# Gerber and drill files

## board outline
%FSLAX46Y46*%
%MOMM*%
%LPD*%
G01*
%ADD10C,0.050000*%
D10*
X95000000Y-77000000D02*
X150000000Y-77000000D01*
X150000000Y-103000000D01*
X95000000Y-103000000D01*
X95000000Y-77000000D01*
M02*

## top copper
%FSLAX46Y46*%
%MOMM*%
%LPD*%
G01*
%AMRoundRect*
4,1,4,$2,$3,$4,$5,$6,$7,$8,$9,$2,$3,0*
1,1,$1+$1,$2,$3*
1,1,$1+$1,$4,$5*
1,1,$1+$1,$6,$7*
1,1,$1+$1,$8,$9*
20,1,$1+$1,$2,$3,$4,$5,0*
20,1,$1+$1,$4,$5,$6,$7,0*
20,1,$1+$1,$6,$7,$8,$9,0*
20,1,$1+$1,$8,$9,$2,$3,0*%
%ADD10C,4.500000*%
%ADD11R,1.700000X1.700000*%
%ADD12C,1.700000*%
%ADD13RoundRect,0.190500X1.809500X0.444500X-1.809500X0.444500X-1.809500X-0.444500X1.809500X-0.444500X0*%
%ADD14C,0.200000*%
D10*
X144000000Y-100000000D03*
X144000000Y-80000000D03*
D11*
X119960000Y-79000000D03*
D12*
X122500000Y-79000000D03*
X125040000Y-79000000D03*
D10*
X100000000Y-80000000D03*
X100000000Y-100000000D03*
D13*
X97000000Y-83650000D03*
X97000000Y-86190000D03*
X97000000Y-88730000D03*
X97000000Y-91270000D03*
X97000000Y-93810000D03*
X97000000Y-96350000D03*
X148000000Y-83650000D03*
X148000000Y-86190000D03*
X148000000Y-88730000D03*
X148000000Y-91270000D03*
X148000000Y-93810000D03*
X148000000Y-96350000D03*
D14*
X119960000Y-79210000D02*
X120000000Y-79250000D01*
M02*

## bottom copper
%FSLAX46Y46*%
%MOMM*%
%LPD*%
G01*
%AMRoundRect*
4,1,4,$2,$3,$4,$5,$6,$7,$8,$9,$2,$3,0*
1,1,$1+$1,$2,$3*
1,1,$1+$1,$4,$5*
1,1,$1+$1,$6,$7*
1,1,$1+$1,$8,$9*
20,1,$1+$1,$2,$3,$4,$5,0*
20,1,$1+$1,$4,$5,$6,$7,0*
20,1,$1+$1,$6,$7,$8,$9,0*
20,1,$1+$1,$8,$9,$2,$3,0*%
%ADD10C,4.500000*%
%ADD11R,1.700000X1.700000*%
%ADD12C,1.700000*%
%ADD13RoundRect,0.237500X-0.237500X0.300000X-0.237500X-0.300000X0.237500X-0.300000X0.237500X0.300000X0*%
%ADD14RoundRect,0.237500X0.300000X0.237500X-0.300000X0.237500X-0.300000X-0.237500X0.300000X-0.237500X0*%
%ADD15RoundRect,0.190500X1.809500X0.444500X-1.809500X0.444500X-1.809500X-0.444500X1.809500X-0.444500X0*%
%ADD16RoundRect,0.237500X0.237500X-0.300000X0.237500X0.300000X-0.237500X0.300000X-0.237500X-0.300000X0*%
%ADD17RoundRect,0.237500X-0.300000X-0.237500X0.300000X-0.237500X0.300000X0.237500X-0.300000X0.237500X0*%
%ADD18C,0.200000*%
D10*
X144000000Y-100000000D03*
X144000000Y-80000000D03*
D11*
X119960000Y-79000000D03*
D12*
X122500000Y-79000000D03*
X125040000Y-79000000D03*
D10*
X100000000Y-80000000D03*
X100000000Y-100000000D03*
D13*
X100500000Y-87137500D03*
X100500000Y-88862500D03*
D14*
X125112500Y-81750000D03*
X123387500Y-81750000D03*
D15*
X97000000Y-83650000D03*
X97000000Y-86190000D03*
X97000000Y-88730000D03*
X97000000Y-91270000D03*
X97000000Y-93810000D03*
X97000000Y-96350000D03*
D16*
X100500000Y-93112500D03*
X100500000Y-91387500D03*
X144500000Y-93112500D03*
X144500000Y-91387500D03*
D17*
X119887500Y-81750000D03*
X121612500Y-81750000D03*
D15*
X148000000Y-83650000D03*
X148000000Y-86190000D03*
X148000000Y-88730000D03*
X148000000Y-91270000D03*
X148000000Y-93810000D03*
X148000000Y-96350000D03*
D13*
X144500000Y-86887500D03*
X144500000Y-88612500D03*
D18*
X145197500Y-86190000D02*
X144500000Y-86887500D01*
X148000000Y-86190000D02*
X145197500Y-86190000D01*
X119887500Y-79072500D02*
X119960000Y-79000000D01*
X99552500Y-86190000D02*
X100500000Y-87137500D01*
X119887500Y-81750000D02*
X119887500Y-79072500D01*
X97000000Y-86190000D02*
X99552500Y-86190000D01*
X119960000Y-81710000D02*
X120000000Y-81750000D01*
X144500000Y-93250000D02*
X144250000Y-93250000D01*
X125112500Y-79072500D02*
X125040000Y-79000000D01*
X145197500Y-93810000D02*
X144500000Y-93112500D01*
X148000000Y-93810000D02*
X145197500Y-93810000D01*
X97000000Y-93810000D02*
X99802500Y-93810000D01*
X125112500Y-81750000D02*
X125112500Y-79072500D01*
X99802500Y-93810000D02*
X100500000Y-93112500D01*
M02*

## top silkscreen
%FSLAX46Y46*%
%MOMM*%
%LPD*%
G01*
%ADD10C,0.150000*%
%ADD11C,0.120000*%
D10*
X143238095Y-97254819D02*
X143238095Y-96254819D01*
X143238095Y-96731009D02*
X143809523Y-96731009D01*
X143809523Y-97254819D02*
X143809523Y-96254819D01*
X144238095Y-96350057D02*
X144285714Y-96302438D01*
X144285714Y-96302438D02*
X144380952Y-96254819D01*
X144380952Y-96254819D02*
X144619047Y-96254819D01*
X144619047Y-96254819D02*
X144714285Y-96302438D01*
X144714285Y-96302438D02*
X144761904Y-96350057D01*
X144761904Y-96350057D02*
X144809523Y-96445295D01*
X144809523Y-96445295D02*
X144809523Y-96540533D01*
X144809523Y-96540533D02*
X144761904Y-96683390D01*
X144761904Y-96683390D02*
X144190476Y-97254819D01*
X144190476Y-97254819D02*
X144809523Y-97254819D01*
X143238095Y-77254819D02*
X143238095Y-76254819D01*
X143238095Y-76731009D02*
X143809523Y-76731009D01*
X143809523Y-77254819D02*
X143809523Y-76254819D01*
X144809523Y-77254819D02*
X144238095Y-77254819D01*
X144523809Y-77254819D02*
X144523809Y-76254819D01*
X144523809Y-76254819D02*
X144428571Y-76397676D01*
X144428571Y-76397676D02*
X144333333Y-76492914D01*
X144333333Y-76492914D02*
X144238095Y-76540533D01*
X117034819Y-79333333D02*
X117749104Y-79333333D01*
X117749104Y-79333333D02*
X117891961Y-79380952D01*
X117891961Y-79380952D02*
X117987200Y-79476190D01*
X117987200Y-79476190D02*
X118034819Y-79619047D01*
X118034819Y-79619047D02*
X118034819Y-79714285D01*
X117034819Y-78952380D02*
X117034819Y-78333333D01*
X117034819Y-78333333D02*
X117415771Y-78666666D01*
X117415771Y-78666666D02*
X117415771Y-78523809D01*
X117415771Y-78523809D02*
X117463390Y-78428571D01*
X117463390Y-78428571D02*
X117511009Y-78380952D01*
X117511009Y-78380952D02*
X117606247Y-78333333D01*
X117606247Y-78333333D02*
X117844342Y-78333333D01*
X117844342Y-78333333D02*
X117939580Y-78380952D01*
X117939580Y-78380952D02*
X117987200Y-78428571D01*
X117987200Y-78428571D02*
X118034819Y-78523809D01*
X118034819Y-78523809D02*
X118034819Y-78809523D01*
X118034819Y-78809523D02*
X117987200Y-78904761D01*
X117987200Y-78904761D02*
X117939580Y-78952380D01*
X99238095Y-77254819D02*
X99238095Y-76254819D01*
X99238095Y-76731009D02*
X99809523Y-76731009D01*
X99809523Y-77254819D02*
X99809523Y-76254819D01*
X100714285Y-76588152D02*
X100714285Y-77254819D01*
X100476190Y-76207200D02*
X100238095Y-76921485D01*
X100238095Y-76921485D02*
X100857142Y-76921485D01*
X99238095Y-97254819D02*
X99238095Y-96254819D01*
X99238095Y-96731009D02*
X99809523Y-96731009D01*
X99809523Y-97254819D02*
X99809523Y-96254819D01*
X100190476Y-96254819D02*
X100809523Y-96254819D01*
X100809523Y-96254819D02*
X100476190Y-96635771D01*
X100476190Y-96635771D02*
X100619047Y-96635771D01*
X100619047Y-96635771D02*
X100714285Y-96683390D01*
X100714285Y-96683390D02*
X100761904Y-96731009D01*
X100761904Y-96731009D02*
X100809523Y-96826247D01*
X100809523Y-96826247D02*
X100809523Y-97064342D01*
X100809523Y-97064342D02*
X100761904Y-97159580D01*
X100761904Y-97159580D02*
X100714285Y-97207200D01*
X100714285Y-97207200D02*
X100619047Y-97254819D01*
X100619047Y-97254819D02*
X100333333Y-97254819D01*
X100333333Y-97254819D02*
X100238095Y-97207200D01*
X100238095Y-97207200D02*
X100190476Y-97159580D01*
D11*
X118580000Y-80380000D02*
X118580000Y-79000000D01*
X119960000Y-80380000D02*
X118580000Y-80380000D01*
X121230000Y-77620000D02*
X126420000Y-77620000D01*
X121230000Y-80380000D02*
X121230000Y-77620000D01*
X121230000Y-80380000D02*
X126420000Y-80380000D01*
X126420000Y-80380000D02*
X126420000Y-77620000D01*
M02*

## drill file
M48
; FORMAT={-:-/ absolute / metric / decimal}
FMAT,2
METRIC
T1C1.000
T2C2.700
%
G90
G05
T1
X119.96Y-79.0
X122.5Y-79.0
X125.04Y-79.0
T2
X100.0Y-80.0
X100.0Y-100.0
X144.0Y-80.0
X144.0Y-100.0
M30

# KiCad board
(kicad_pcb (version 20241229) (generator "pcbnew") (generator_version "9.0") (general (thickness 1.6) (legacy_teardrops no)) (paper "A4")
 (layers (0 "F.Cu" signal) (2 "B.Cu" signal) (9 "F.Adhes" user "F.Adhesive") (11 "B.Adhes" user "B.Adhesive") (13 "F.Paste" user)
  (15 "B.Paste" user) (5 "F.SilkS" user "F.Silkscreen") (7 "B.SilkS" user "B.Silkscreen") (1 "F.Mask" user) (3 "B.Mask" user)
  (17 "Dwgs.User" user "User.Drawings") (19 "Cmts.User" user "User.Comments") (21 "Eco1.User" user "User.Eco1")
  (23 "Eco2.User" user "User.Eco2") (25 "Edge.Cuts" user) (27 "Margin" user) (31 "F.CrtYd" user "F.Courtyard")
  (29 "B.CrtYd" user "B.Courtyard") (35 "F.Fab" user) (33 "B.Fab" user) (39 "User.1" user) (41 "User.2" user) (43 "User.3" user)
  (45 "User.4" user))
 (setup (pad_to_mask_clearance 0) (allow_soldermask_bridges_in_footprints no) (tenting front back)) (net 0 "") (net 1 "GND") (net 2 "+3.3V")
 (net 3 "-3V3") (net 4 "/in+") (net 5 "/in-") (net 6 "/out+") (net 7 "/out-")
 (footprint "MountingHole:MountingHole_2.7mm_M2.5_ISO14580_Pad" (layer "F.Cu") (at 144 100)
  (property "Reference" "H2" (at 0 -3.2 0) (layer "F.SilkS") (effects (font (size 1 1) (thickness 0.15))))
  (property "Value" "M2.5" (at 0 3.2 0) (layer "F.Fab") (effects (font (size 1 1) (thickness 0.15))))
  (pad "1" thru_hole circle (at 0 0) (size 4.5 4.5) (drill 2.7) (layers "*.Cu" "*.Mask") (remove_unused_layers no) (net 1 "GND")
   (zone_connect 2)))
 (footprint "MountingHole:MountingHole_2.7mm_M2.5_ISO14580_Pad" (layer "F.Cu") (at 144 80)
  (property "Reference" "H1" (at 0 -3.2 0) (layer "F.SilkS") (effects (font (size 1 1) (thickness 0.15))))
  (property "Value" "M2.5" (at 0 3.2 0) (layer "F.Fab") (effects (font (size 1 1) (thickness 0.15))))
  (pad "1" thru_hole circle (at 0 0) (size 4.5 4.5) (drill 2.7) (layers "*.Cu" "*.Mask") (remove_unused_layers no) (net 1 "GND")
   (zone_connect 2)))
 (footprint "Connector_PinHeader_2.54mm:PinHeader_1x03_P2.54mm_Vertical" (layer "F.Cu") (at 119.96 79 90)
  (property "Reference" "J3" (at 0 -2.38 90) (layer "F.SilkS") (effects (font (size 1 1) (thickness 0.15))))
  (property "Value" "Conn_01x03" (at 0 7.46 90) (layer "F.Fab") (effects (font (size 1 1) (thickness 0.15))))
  (fp_line (start -1.38 -1.38) (end 0 -1.38) (stroke (width 0.12) (type solid)) (layer "F.SilkS"))
  (fp_line (start -1.38 0) (end -1.38 -1.38) (stroke (width 0.12) (type solid)) (layer "F.SilkS"))
  (fp_line (start 1.38 1.27) (end 1.38 6.46) (stroke (width 0.12) (type solid)) (layer "F.SilkS"))
  (fp_line (start -1.38 1.27) (end 1.38 1.27) (stroke (width 0.12) (type solid)) (layer "F.SilkS"))
  (fp_line (start -1.38 1.27) (end -1.38 6.46) (stroke (width 0.12) (type solid)) (layer "F.SilkS"))
  (fp_line (start -1.38 6.46) (end 1.38 6.46) (stroke (width 0.12) (type solid)) (layer "F.SilkS"))
  (pad "1" thru_hole rect (at 0 0 90) (size 1.7 1.7) (drill 1) (layers "*.Cu" "*.Mask") (remove_unused_layers no) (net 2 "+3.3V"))
  (pad "2" thru_hole circle (at 0 2.54 90) (size 1.7 1.7) (drill 1) (layers "*.Cu" "*.Mask") (remove_unused_layers no) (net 1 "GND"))
  (pad "3" thru_hole circle (at 0 5.08 90) (size 1.7 1.7) (drill 1) (layers "*.Cu" "*.Mask") (remove_unused_layers no) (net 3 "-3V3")))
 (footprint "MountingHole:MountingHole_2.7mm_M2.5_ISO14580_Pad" (layer "F.Cu") (at 100 80)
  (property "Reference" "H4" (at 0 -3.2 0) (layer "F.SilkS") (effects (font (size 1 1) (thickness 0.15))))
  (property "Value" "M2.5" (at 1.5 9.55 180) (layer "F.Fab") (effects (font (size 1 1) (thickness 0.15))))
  (pad "1" thru_hole circle (at 0 0) (size 4.5 4.5) (drill 2.7) (layers "*.Cu" "*.Mask") (remove_unused_layers no) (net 1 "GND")
   (zone_connect 2)))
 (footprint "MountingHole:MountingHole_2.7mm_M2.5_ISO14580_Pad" (layer "F.Cu") (at 100 100)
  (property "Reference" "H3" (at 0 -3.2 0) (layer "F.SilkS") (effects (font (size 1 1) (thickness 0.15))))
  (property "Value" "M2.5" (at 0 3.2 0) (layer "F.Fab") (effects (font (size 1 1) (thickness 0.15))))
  (pad "1" thru_hole circle (at 0 0) (size 4.5 4.5) (drill 2.7) (layers "*.Cu" "*.Mask") (remove_unused_layers no) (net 1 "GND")
   (zone_connect 2)))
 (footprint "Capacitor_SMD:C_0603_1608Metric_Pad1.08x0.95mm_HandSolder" (layer "B.Cu") (at 100.5 88 -90)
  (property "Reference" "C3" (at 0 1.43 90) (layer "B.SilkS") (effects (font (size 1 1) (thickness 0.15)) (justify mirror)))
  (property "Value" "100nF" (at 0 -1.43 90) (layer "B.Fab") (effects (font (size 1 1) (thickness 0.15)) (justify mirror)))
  (pad "1" smd roundrect (at -0.8625 0 270) (size 1.075 0.95) (layers "B.Cu" "B.Mask" "B.Paste") (roundrect_rratio 0.25) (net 2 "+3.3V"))
  (pad "2" smd roundrect (at 0.8625 0 270) (size 1.075 0.95) (layers "B.Cu" "B.Mask" "B.Paste") (roundrect_rratio 0.25) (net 1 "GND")))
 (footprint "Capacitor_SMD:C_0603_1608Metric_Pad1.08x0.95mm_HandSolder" (layer "B.Cu") (at 124.25 81.75 180)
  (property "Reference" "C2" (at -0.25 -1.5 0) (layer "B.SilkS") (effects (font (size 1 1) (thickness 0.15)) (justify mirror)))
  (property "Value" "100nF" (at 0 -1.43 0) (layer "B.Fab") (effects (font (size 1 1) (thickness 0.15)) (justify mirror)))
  (pad "1" smd roundrect (at -0.8625 0 180) (size 1.075 0.95) (layers "B.Cu" "B.Mask" "B.Paste") (roundrect_rratio 0.25) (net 3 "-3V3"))
  (pad "2" smd roundrect (at 0.8625 0 180) (size 1.075 0.95) (layers "B.Cu" "B.Mask" "B.Paste") (roundrect_rratio 0.25) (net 1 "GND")))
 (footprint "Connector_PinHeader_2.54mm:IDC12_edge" (layer "B.Cu") (at 97 83.65 180)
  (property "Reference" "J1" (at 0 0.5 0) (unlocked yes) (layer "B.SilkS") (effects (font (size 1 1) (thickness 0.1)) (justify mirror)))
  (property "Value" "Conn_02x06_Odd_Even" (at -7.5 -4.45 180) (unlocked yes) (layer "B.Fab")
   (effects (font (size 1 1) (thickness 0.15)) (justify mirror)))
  (pad "1" smd roundrect (at 0 0 180) (size 4 1.27) (layers "B.Cu" "B.Mask" "B.Paste") (roundrect_rratio 0.15) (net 1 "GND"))
  (pad "2" smd roundrect (at 0 0 180) (size 4 1.27) (layers "F.Cu" "F.Mask" "F.Paste") (roundrect_rratio 0.15) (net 1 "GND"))
  (pad "3" smd roundrect (at 0 -2.54 180) (size 4 1.27) (layers "B.Cu" "B.Mask" "B.Paste") (roundrect_rratio 0.15) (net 2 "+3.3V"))
  (pad "4" smd roundrect (at 0 -2.54 180) (size 4 1.27) (layers "F.Cu" "F.Mask" "F.Paste") (roundrect_rratio 0.15) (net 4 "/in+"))
  (pad "5" smd roundrect (at 0 -5.08 180) (size 4 1.27) (layers "B.Cu" "B.Mask" "B.Paste") (roundrect_rratio 0.15) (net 1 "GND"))
  (pad "6" smd roundrect (at 0 -5.08 180) (size 4 1.27) (layers "F.Cu" "F.Mask" "F.Paste") (roundrect_rratio 0.15) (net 1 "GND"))
  (pad "7" smd roundrect (at 0 -7.62 180) (size 4 1.27) (layers "B.Cu" "B.Mask" "B.Paste") (roundrect_rratio 0.15) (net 1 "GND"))
  (pad "8" smd roundrect (at 0 -7.62 180) (size 4 1.27) (layers "F.Cu" "F.Mask" "F.Paste") (roundrect_rratio 0.15) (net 1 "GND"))
  (pad "9" smd roundrect (at 0 -10.16 180) (size 4 1.27) (layers "B.Cu" "B.Mask" "B.Paste") (roundrect_rratio 0.15) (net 3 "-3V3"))
  (pad "10" smd roundrect (at 0 -10.16 180) (size 4 1.27) (layers "F.Cu" "F.Mask" "F.Paste") (roundrect_rratio 0.15) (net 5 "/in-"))
  (pad "11" smd roundrect (at 0 -12.7 180) (size 4 1.27) (layers "B.Cu" "B.Mask" "B.Paste") (roundrect_rratio 0.15) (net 1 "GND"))
  (pad "12" smd roundrect (at 0 -12.7 180) (size 4 1.27) (layers "F.Cu" "F.Mask" "F.Paste") (roundrect_rratio 0.15) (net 1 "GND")))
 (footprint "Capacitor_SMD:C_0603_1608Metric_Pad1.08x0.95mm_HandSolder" (layer "B.Cu") (at 100.5 92.25 90)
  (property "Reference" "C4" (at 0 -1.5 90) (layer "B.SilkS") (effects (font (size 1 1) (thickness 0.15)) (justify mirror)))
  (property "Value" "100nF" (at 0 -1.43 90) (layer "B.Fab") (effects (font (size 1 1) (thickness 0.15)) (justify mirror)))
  (pad "1" smd roundrect (at -0.8625 0 90) (size 1.075 0.95) (layers "B.Cu" "B.Mask" "B.Paste") (roundrect_rratio 0.25) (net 3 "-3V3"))
  (pad "2" smd roundrect (at 0.8625 0 90) (size 1.075 0.95) (layers "B.Cu" "B.Mask" "B.Paste") (roundrect_rratio 0.25) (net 1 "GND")))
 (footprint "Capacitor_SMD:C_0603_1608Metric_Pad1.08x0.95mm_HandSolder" (layer "B.Cu") (at 144.5 92.25 90)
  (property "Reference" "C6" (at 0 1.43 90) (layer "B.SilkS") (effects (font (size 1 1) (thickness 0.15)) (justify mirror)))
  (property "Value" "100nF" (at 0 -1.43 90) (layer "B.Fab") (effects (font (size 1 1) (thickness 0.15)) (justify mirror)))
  (pad "1" smd roundrect (at -0.8625 0 90) (size 1.075 0.95) (layers "B.Cu" "B.Mask" "B.Paste") (roundrect_rratio 0.25) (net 3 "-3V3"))
  (pad "2" smd roundrect (at 0.8625 0 90) (size 1.075 0.95) (layers "B.Cu" "B.Mask" "B.Paste") (roundrect_rratio 0.25) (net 1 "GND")))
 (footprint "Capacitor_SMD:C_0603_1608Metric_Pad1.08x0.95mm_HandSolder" (layer "B.Cu") (at 120.75 81.75)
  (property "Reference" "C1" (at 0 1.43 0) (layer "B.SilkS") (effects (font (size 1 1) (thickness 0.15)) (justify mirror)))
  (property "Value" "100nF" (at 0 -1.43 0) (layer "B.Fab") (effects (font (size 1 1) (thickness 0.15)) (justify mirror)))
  (pad "1" smd roundrect (at -0.8625 0) (size 1.075 0.95) (layers "B.Cu" "B.Mask" "B.Paste") (roundrect_rratio 0.25) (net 2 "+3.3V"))
  (pad "2" smd roundrect (at 0.8625 0) (size 1.075 0.95) (layers "B.Cu" "B.Mask" "B.Paste") (roundrect_rratio 0.25) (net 1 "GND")))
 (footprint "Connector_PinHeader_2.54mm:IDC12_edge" (layer "B.Cu") (at 148 83.65 180)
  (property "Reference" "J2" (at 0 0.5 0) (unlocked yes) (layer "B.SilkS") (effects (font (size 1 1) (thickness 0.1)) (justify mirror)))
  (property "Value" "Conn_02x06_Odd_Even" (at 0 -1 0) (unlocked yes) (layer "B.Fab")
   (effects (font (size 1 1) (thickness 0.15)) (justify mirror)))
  (pad "1" smd roundrect (at 0 0 180) (size 4 1.27) (layers "B.Cu" "B.Mask" "B.Paste") (roundrect_rratio 0.15) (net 1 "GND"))
  (pad "2" smd roundrect (at 0 0 180) (size 4 1.27) (layers "F.Cu" "F.Mask" "F.Paste") (roundrect_rratio 0.15) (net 1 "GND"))
  (pad "3" smd roundrect (at 0 -2.54 180) (size 4 1.27) (layers "B.Cu" "B.Mask" "B.Paste") (roundrect_rratio 0.15) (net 2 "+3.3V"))
  (pad "4" smd roundrect (at 0 -2.54 180) (size 4 1.27) (layers "F.Cu" "F.Mask" "F.Paste") (roundrect_rratio 0.15) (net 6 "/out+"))
  (pad "5" smd roundrect (at 0 -5.08 180) (size 4 1.27) (layers "B.Cu" "B.Mask" "B.Paste") (roundrect_rratio 0.15) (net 1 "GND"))
  (pad "6" smd roundrect (at 0 -5.08 180) (size 4 1.27) (layers "F.Cu" "F.Mask" "F.Paste") (roundrect_rratio 0.15) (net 1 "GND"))
  (pad "7" smd roundrect (at 0 -7.62 180) (size 4 1.27) (layers "B.Cu" "B.Mask" "B.Paste") (roundrect_rratio 0.15) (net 1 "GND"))
  (pad "8" smd roundrect (at 0 -7.62 180) (size 4 1.27) (layers "F.Cu" "F.Mask" "F.Paste") (roundrect_rratio 0.15) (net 1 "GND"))
  (pad "9" smd roundrect (at 0 -10.16 180) (size 4 1.27) (layers "B.Cu" "B.Mask" "B.Paste") (roundrect_rratio 0.15) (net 3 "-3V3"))
  (pad "10" smd roundrect (at 0 -10.16 180) (size 4 1.27) (layers "F.Cu" "F.Mask" "F.Paste") (roundrect_rratio 0.15) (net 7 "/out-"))
  (pad "11" smd roundrect (at 0 -12.7 180) (size 4 1.27) (layers "B.Cu" "B.Mask" "B.Paste") (roundrect_rratio 0.15) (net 1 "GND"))
  (pad "12" smd roundrect (at 0 -12.7 180) (size 4 1.27) (layers "F.Cu" "F.Mask" "F.Paste") (roundrect_rratio 0.15) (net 1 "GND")))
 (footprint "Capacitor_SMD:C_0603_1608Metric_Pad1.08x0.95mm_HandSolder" (layer "B.Cu") (at 144.5 87.75 -90)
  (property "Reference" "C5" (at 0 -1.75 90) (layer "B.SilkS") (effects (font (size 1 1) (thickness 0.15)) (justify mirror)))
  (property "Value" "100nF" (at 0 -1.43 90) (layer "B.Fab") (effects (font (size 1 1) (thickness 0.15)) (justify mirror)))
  (pad "1" smd roundrect (at -0.8625 0 270) (size 1.075 0.95) (layers "B.Cu" "B.Mask" "B.Paste") (roundrect_rratio 0.25) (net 2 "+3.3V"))
  (pad "2" smd roundrect (at 0.8625 0 270) (size 1.075 0.95) (layers "B.Cu" "B.Mask" "B.Paste") (roundrect_rratio 0.25) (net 1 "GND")))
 (gr_rect (start 95 77) (end 150 103) (stroke (width 0.05) (type default)) (fill no) (layer "Edge.Cuts"))
 (segment (start 119.96 79.21) (end 120 79.25) (width 0.2) (layer "F.Cu") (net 2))
 (segment (start 145.1975 86.19) (end 144.5 86.8875) (width 0.2) (layer "B.Cu") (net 2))
 (segment (start 148 86.19) (end 145.1975 86.19) (width 0.2) (layer "B.Cu") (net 2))
 (segment (start 119.8875 79.0725) (end 119.96 79) (width 0.2) (layer "B.Cu") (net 2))
 (segment (start 99.5525 86.19) (end 100.5 87.1375) (width 0.2) (layer "B.Cu") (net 2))
 (segment (start 119.8875 81.75) (end 119.8875 79.0725) (width 0.2) (layer "B.Cu") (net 2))
 (segment (start 97 86.19) (end 99.5525 86.19) (width 0.2) (layer "B.Cu") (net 2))
 (segment (start 119.96 81.71) (end 120 81.75) (width 0.2) (layer "B.Cu") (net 2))
 (segment (start 144.5 93.25) (end 144.25 93.25) (width 0.2) (layer "B.Cu") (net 3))
 (segment (start 125.1125 79.0725) (end 125.04 79) (width 0.2) (layer "B.Cu") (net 3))
 (segment (start 145.1975 93.81) (end 144.5 93.1125) (width 0.2) (layer "B.Cu") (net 3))
 (segment (start 148 93.81) (end 145.1975 93.81) (width 0.2) (layer "B.Cu") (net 3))
 (segment (start 97 93.81) (end 99.8025 93.81) (width 0.2) (layer "B.Cu") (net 3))
 (segment (start 125.1125 81.75) (end 125.1125 79.0725) (width 0.2) (layer "B.Cu") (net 3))
 (segment (start 99.8025 93.81) (end 100.5 93.1125) (width 0.2) (layer "B.Cu") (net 3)))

